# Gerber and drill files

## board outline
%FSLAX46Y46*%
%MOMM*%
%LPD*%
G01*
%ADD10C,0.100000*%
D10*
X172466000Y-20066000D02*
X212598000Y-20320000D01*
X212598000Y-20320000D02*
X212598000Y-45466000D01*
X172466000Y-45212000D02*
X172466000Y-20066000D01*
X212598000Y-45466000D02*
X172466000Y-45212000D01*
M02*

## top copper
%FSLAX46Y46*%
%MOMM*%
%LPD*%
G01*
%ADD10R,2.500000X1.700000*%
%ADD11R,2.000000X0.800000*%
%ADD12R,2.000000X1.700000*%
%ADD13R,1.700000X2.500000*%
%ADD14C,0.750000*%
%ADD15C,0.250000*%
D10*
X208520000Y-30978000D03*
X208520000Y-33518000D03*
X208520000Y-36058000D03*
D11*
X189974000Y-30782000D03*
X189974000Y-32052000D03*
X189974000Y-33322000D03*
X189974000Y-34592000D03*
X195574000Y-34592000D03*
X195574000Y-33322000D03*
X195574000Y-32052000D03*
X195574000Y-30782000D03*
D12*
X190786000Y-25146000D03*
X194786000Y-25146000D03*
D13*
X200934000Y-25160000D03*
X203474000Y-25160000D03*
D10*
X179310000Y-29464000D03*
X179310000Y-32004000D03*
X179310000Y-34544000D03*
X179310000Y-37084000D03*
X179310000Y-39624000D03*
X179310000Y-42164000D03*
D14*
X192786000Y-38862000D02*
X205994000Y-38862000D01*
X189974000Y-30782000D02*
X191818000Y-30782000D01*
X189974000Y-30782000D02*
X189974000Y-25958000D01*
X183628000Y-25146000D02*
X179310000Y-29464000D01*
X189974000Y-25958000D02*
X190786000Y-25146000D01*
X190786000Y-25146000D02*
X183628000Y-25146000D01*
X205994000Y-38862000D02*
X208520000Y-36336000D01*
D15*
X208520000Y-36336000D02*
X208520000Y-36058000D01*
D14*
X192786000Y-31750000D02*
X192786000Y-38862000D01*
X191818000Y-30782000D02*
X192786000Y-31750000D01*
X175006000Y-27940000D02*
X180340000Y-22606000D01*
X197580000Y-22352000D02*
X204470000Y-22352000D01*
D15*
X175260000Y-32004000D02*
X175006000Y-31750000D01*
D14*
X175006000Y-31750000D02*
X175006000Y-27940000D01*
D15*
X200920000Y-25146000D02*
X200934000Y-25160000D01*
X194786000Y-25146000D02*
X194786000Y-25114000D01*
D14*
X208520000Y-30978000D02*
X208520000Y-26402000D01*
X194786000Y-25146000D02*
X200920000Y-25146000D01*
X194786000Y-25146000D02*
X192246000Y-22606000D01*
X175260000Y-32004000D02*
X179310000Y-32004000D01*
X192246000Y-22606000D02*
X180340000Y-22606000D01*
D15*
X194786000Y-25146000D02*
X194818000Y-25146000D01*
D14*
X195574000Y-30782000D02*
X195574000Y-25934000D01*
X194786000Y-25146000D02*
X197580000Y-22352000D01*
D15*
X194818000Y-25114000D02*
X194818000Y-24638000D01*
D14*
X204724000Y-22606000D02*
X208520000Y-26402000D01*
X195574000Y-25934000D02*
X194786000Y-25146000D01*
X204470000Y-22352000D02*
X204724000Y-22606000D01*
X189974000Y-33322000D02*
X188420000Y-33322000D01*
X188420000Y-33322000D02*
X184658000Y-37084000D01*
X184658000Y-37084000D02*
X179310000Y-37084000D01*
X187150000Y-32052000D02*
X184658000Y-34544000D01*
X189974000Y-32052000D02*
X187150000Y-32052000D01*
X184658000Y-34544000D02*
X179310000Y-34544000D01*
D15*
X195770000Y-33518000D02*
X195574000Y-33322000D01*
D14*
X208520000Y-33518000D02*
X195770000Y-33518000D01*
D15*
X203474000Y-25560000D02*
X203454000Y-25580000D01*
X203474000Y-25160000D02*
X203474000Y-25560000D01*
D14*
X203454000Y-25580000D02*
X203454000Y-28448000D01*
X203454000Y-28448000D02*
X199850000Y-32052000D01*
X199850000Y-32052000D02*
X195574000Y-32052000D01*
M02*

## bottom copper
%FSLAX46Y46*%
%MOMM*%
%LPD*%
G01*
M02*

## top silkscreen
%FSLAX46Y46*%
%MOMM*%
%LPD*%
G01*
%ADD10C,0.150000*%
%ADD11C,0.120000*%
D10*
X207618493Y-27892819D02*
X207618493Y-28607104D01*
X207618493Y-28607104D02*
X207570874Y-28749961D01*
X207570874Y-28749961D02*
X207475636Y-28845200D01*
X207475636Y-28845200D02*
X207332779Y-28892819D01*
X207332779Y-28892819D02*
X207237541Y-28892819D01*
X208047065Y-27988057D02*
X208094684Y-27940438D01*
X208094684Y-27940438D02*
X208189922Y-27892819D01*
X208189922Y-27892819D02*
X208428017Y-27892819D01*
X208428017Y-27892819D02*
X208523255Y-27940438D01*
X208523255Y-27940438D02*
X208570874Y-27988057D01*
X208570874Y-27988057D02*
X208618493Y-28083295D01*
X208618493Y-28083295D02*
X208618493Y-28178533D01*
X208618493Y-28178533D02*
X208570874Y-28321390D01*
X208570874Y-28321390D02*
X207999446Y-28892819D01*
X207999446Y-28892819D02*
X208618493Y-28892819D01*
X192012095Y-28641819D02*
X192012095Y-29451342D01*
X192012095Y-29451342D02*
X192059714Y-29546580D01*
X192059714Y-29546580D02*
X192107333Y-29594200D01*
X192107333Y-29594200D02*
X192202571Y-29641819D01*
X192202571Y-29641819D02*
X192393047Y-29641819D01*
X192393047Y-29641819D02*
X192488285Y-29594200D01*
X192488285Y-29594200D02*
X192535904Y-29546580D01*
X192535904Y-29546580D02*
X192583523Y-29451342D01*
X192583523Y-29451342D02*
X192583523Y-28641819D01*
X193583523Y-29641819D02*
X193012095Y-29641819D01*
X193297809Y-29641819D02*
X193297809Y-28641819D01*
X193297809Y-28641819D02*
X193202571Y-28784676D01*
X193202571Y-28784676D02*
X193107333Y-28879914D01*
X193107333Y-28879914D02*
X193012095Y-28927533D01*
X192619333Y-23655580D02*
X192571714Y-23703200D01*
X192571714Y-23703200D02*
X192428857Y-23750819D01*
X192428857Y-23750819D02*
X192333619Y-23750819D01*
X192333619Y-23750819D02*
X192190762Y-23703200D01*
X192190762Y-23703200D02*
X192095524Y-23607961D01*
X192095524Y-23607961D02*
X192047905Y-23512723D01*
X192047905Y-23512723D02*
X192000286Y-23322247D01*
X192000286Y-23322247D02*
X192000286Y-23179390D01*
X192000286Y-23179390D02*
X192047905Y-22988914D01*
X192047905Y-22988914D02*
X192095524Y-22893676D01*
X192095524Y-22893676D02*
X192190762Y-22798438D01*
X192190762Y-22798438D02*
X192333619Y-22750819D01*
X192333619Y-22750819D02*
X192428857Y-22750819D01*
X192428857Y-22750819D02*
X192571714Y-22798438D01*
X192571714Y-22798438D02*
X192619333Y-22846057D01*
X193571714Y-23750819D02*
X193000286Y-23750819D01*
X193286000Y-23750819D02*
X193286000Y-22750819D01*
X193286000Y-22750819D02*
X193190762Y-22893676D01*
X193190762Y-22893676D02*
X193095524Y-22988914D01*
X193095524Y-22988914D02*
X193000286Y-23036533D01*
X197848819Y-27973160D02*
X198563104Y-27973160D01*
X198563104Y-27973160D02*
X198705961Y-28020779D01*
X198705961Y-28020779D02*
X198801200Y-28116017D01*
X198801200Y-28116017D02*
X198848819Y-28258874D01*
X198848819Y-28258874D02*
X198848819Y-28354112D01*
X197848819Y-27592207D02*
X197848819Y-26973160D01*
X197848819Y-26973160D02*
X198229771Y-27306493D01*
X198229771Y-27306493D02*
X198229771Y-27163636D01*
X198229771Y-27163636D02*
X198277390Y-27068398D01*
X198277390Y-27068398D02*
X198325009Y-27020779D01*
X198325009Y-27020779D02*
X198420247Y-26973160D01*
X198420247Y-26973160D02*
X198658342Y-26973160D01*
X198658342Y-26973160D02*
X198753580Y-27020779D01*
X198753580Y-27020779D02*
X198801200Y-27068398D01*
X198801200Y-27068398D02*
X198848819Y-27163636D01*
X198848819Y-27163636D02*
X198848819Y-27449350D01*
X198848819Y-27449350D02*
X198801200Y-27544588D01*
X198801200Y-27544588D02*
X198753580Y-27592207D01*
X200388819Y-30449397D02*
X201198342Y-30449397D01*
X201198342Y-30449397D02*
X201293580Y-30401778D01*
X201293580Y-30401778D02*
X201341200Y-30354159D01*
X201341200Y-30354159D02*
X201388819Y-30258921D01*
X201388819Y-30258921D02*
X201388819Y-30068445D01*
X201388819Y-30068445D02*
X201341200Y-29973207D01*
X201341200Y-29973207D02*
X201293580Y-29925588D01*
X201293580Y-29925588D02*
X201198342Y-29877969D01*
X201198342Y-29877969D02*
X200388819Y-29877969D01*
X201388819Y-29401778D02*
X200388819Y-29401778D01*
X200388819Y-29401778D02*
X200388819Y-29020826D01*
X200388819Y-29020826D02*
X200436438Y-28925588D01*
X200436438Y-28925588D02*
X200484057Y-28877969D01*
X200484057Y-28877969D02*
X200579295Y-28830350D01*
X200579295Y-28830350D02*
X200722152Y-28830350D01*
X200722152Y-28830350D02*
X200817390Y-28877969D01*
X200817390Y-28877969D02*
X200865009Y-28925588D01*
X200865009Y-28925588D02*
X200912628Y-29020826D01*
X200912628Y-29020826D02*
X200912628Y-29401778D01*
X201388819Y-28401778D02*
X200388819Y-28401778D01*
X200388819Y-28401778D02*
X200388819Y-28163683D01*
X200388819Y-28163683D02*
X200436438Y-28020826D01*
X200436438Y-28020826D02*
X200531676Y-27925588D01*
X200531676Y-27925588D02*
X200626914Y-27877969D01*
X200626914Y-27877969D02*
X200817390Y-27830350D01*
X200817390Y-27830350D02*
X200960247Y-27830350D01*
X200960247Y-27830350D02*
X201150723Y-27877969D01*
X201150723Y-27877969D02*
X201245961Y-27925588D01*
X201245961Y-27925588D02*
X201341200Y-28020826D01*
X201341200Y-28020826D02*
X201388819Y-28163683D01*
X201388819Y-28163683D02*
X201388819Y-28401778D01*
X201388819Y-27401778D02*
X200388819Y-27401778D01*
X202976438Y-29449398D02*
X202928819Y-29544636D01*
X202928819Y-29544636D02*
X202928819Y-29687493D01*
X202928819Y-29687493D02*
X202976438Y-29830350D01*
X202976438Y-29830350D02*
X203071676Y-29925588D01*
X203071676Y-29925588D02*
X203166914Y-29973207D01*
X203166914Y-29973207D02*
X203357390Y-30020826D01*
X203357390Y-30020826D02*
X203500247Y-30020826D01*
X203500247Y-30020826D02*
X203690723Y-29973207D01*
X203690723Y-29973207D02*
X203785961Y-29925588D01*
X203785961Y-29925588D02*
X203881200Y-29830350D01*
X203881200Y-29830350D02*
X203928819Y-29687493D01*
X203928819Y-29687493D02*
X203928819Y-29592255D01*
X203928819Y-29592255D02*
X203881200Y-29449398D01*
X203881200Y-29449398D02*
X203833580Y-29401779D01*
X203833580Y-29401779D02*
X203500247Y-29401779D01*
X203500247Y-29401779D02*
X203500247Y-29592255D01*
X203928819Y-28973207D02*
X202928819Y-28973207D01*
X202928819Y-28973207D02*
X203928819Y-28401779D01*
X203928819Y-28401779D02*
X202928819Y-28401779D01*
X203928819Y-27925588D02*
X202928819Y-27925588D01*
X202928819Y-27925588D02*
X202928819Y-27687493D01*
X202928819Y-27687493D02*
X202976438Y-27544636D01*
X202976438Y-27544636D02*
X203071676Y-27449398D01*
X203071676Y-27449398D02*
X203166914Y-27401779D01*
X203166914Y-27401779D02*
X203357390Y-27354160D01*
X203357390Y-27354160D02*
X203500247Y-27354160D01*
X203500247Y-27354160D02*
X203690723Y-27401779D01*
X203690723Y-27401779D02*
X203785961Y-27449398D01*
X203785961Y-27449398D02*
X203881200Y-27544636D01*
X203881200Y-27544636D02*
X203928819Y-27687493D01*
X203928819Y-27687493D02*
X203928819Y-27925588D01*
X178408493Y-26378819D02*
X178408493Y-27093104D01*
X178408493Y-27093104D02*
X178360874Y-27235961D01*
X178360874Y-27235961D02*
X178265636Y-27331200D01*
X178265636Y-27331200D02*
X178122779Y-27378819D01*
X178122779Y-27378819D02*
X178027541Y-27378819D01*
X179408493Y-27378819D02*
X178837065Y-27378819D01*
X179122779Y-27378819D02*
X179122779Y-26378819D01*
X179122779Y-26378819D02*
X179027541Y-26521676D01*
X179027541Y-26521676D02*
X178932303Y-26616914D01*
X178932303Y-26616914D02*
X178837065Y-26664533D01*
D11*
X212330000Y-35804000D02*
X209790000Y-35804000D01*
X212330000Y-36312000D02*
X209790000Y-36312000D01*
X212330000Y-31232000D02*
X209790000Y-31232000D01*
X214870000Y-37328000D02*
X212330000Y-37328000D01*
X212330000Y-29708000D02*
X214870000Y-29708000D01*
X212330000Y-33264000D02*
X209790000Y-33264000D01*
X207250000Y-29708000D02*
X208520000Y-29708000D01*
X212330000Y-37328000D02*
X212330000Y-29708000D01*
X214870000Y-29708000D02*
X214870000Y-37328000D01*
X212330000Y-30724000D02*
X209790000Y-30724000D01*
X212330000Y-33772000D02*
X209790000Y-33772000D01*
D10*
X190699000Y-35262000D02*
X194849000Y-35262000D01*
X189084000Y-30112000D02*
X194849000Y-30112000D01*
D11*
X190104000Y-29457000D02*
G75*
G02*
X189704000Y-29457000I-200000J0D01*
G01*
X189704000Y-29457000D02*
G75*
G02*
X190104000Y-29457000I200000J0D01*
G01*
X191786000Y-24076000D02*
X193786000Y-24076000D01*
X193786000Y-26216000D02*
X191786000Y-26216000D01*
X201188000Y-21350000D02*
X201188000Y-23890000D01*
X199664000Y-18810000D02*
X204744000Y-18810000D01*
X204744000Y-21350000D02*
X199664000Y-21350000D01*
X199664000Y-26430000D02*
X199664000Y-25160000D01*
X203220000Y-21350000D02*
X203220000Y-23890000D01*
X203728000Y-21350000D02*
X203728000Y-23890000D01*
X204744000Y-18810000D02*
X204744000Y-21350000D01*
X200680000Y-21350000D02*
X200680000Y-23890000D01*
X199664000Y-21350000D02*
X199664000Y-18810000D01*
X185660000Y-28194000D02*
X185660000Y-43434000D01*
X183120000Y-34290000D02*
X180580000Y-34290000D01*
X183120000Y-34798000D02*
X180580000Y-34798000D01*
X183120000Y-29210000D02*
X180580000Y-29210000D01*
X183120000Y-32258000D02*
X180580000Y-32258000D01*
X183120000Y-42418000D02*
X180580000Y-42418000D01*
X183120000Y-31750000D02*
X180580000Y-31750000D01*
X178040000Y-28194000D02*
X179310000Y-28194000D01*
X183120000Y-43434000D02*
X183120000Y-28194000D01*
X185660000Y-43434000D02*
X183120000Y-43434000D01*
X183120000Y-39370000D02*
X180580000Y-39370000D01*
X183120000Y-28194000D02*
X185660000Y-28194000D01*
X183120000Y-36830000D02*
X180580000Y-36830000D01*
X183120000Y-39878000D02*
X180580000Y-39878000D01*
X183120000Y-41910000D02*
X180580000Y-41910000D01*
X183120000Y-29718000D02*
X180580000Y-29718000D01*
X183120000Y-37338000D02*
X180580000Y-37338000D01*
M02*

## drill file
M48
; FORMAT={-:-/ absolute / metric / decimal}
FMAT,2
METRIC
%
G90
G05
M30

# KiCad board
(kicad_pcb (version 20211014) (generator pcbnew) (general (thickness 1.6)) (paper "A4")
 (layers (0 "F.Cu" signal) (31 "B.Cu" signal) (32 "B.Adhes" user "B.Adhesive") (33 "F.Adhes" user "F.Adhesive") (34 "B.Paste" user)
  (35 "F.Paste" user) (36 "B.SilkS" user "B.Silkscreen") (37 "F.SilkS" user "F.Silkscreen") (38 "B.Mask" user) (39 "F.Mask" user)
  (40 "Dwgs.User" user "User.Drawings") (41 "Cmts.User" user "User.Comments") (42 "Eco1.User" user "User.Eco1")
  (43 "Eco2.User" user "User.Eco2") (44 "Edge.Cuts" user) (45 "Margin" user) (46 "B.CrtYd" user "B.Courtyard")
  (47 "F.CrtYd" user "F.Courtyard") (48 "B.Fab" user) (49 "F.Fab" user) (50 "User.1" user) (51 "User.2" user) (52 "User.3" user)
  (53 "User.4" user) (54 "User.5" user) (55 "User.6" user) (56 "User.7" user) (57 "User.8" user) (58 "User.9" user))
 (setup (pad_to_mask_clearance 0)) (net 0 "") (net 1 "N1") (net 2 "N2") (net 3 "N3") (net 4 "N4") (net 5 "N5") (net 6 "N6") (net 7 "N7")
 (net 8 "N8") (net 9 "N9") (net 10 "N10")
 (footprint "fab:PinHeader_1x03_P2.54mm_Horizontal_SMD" (layer "F.Cu") (at 208.52 30.978)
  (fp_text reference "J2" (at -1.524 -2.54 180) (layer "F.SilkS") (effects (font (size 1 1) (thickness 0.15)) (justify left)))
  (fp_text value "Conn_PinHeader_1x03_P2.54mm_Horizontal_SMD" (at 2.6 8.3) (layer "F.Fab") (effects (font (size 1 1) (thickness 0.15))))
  (fp_line (start 3.81 4.826) (end 1.27 4.826) (layer "F.SilkS") (width 0.12))
  (fp_line (start 3.81 5.334) (end 1.27 5.334) (layer "F.SilkS") (width 0.12))
  (fp_line (start 3.81 0.254) (end 1.27 0.254) (layer "F.SilkS") (width 0.12))
  (fp_line (start 6.35 6.35) (end 3.81 6.35) (layer "F.SilkS") (width 0.12))
  (fp_line (start 3.81 -1.27) (end 6.35 -1.27) (layer "F.SilkS") (width 0.12))
  (fp_line (start 3.81 2.286) (end 1.27 2.286) (layer "F.SilkS") (width 0.12))
  (fp_line (start -1.27 -1.27) (end 0 -1.27) (layer "F.SilkS") (width 0.12))
  (fp_line (start 3.81 6.35) (end 3.81 -1.27) (layer "F.SilkS") (width 0.12))
  (fp_line (start 6.35 -1.27) (end 6.35 6.35) (layer "F.SilkS") (width 0.12))
  (fp_line (start 3.81 -0.254) (end 1.27 -0.254) (layer "F.SilkS") (width 0.12))
  (fp_line (start 3.81 2.794) (end 1.27 2.794) (layer "F.SilkS") (width 0.12))
  (pad "1" smd rect locked (at 0 0) (size 2.5 1.7) (layers "F.Cu" "F.Paste" "F.Mask") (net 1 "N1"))
  (pad "2" smd rect locked (at 0 2.54) (size 2.5 1.7) (layers "F.Cu" "F.Paste" "F.Mask") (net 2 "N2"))
  (pad "3" smd rect locked (at 0 5.08) (size 2.5 1.7) (layers "F.Cu" "F.Paste" "F.Mask") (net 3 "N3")))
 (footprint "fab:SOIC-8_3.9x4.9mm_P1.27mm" (layer "F.Cu") (at 192.774 32.687)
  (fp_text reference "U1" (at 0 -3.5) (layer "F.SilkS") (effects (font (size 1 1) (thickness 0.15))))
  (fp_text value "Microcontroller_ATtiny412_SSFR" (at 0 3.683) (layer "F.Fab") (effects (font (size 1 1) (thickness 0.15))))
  (fp_line (start -2.075 2.575) (end 2.075 2.575) (layer "F.SilkS") (width 0.15))
  (fp_line (start -3.69 -2.575) (end 2.075 -2.575) (layer "F.SilkS") (width 0.15))
  (fp_circle (center -2.87 -3.23) (end -2.67 -3.23) (layer "F.SilkS") (width 0.12) (fill none))
  (pad "1" smd rect locked (at -2.8 -1.905) (size 2 0.8) (layers "F.Cu" "F.Paste" "F.Mask") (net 3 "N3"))
  (pad "2" smd rect locked (at -2.8 -0.635) (size 2 0.8) (layers "F.Cu" "F.Paste" "F.Mask") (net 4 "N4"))
  (pad "3" smd rect locked (at -2.8 0.635) (size 2 0.8) (layers "F.Cu" "F.Paste" "F.Mask") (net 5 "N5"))
  (pad "4" smd rect locked (at -2.8 1.905) (size 2 0.8) (layers "F.Cu" "F.Paste" "F.Mask") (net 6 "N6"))
  (pad "5" smd rect locked (at 2.8 1.905) (size 2 0.8) (layers "F.Cu" "F.Paste" "F.Mask") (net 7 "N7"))
  (pad "6" smd rect locked (at 2.8 0.635) (size 2 0.8) (layers "F.Cu" "F.Paste" "F.Mask") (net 2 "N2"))
  (pad "7" smd rect locked (at 2.8 -0.635) (size 2 0.8) (layers "F.Cu" "F.Paste" "F.Mask") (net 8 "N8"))
  (pad "8" smd rect locked (at 2.8 -1.905) (size 2 0.8) (layers "F.Cu" "F.Paste" "F.Mask") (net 1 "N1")))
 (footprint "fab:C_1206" (layer "F.Cu") (at 192.786 25.146)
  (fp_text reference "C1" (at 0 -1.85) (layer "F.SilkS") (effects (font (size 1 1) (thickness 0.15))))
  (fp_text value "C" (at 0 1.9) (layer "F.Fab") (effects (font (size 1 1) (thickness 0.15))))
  (fp_line (start -1 -1.07) (end 1 -1.07) (layer "F.SilkS") (width 0.12))
  (fp_line (start 1 1.07) (end -1 1.07) (layer "F.SilkS") (width 0.12))
  (pad "1" smd rect locked (at -2 0) (size 2 1.7) (layers "F.Cu" "F.Paste" "F.Mask") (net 3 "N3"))
  (pad "2" smd rect locked (at 2 0) (size 2 1.7) (layers "F.Cu" "F.Paste" "F.Mask") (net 1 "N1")))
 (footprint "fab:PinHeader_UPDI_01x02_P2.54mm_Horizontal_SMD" (layer "F.Cu") (at 200.934 25.16 90)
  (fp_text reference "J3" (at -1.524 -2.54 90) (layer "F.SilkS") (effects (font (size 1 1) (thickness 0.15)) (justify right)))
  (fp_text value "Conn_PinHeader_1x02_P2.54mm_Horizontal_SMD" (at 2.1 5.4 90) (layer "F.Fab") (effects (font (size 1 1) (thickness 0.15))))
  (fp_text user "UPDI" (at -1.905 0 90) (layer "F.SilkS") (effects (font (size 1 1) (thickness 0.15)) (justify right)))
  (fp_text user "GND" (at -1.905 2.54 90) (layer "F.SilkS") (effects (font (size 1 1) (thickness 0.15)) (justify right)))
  (fp_line (start 3.81 0.254) (end 1.27 0.254) (layer "F.SilkS") (width 0.12))
  (fp_line (start 6.35 -1.27) (end 6.35 3.81) (layer "F.SilkS") (width 0.12))
  (fp_line (start 3.81 3.81) (end 3.81 -1.27) (layer "F.SilkS") (width 0.12))
  (fp_line (start -1.27 -1.27) (end 0 -1.27) (layer "F.SilkS") (width 0.12))
  (fp_line (start 3.81 2.286) (end 1.27 2.286) (layer "F.SilkS") (width 0.12))
  (fp_line (start 3.81 2.794) (end 1.27 2.794) (layer "F.SilkS") (width 0.12))
  (fp_line (start 6.35 3.81) (end 3.81 3.81) (layer "F.SilkS") (width 0.12))
  (fp_line (start 3.81 -0.254) (end 1.27 -0.254) (layer "F.SilkS") (width 0.12))
  (fp_line (start 3.81 -1.27) (end 6.35 -1.27) (layer "F.SilkS") (width 0.12))
  (pad "1" smd rect locked (at 0 0 90) (size 2.5 1.7) (layers "F.Cu" "F.Paste" "F.Mask") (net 1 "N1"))
  (pad "2" smd rect locked (at 0 2.54 90) (size 2.5 1.7) (layers "F.Cu" "F.Paste" "F.Mask") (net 8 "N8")))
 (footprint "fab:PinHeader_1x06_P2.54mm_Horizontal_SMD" (layer "F.Cu") (at 179.31 29.464)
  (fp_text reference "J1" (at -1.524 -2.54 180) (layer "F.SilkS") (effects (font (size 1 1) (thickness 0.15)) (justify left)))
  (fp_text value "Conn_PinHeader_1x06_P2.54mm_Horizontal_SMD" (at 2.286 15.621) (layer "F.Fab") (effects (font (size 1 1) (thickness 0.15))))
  (fp_line (start 6.35 -1.27) (end 6.35 13.97) (layer "F.SilkS") (width 0.12))
  (fp_line (start 3.81 4.826) (end 1.27 4.826) (layer "F.SilkS") (width 0.12))
  (fp_line (start 3.81 5.334) (end 1.27 5.334) (layer "F.SilkS") (width 0.12))
  (fp_line (start 3.81 -0.254) (end 1.27 -0.254) (layer "F.SilkS") (width 0.12))
  (fp_line (start 3.81 2.794) (end 1.27 2.794) (layer "F.SilkS") (width 0.12))
  (fp_line (start 3.81 12.954) (end 1.27 12.954) (layer "F.SilkS") (width 0.12))
  (fp_line (start 3.81 2.286) (end 1.27 2.286) (layer "F.SilkS") (width 0.12))
  (fp_line (start -1.27 -1.27) (end 0 -1.27) (layer "F.SilkS") (width 0.12))
  (fp_line (start 3.81 13.97) (end 3.81 -1.27) (layer "F.SilkS") (width 0.12))
  (fp_line (start 6.35 13.97) (end 3.81 13.97) (layer "F.SilkS") (width 0.12))
  (fp_line (start 3.81 9.906) (end 1.27 9.906) (layer "F.SilkS") (width 0.12))
  (fp_line (start 3.81 -1.27) (end 6.35 -1.27) (layer "F.SilkS") (width 0.12))
  (fp_line (start 3.81 7.366) (end 1.27 7.366) (layer "F.SilkS") (width 0.12))
  (fp_line (start 3.81 10.414) (end 1.27 10.414) (layer "F.SilkS") (width 0.12))
  (fp_line (start 3.81 12.446) (end 1.27 12.446) (layer "F.SilkS") (width 0.12))
  (fp_line (start 3.81 0.254) (end 1.27 0.254) (layer "F.SilkS") (width 0.12))
  (fp_line (start 3.81 7.874) (end 1.27 7.874) (layer "F.SilkS") (width 0.12))
  (pad "1" smd rect locked (at 0 0) (size 2.5 1.7) (layers "F.Cu" "F.Paste" "F.Mask") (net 3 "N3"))
  (pad "2" smd rect locked (at 0 2.54) (size 2.5 1.7) (layers "F.Cu" "F.Paste" "F.Mask") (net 1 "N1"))
  (pad "3" smd rect locked (at 0 5.08) (size 2.5 1.7) (layers "F.Cu" "F.Paste" "F.Mask") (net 4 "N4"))
  (pad "4" smd rect locked (at 0 7.62) (size 2.5 1.7) (layers "F.Cu" "F.Paste" "F.Mask") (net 5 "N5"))
  (pad "5" smd rect locked (at 0 10.16) (size 2.5 1.7) (layers "F.Cu" "F.Paste" "F.Mask") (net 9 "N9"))
  (pad "6" smd rect locked (at 0 12.7) (size 2.5 1.7) (layers "F.Cu" "F.Paste" "F.Mask") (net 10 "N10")))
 (gr_line (start 172.466 20.066) (end 212.598 20.32) (layer "Edge.Cuts") (width 0.1))
 (gr_line (start 212.598 20.32) (end 212.598 45.466) (layer "Edge.Cuts") (width 0.1))
 (gr_line (start 172.466 45.212) (end 172.466 20.066) (layer "Edge.Cuts") (width 0.1))
 (gr_line (start 212.598 45.466) (end 172.466 45.212) (layer "Edge.Cuts") (width 0.1))
 (segment (start 192.786 38.862) (end 205.994 38.862) (width 0.75) (layer "F.Cu") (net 3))
 (segment (start 189.974 30.782) (end 191.818 30.782) (width 0.75) (layer "F.Cu") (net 3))
 (segment (start 189.974 30.782) (end 189.974 25.958) (width 0.75) (layer "F.Cu") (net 3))
 (segment (start 183.628 25.146) (end 179.31 29.464) (width 0.75) (layer "F.Cu") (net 3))
 (segment (start 189.974 25.958) (end 190.786 25.146) (width 0.75) (layer "F.Cu") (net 3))
 (segment (start 190.786 25.146) (end 183.628 25.146) (width 0.75) (layer "F.Cu") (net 3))
 (segment (start 205.994 38.862) (end 208.52 36.336) (width 0.75) (layer "F.Cu") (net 3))
 (segment (start 208.52 36.336) (end 208.52 36.058) (width 0.25) (layer "F.Cu") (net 3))
 (segment (start 192.786 31.75) (end 192.786 38.862) (width 0.75) (layer "F.Cu") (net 3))
 (segment (start 191.818 30.782) (end 192.786 31.75) (width 0.75) (layer "F.Cu") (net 3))
 (segment (start 175.006 27.94) (end 180.34 22.606) (width 0.75) (layer "F.Cu") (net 1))
 (segment (start 197.58 22.352) (end 204.47 22.352) (width 0.75) (layer "F.Cu") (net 1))
 (segment (start 175.26 32.004) (end 175.006 31.75) (width 0.25) (layer "F.Cu") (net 1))
 (segment (start 175.006 31.75) (end 175.006 27.94) (width 0.75) (layer "F.Cu") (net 1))
 (segment (start 200.92 25.146) (end 200.934 25.16) (width 0.25) (layer "F.Cu") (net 1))
 (segment (start 194.786 25.146) (end 194.786 25.114) (width 0.25) (layer "F.Cu") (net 1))
 (segment (start 208.52 30.978) (end 208.52 26.402) (width 0.75) (layer "F.Cu") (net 1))
 (segment (start 194.786 25.146) (end 200.92 25.146) (width 0.75) (layer "F.Cu") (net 1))
 (segment (start 194.786 25.146) (end 192.246 22.606) (width 0.75) (layer "F.Cu") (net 1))
 (segment (start 175.26 32.004) (end 179.31 32.004) (width 0.75) (layer "F.Cu") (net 1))
 (segment (start 192.246 22.606) (end 180.34 22.606) (width 0.75) (layer "F.Cu") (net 1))
 (segment (start 194.786 25.146) (end 194.818 25.146) (width 0.25) (layer "F.Cu") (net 1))
 (segment (start 195.574 30.782) (end 195.574 25.934) (width 0.75) (layer "F.Cu") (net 1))
 (segment (start 194.786 25.146) (end 197.58 22.352) (width 0.75) (layer "F.Cu") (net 1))
 (segment (start 194.818 25.114) (end 194.818 24.638) (width 0.25) (layer "F.Cu") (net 1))
 (segment (start 204.724 22.606) (end 208.52 26.402) (width 0.75) (layer "F.Cu") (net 1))
 (segment (start 195.574 25.934) (end 194.786 25.146) (width 0.75) (layer "F.Cu") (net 1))
 (segment (start 204.47 22.352) (end 204.724 22.606) (width 0.75) (layer "F.Cu") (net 1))
 (segment (start 189.974 33.322) (end 188.42 33.322) (width 0.75) (layer "F.Cu") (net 5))
 (segment (start 188.42 33.322) (end 184.658 37.084) (width 0.75) (layer "F.Cu") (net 5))
 (segment (start 184.658 37.084) (end 179.31 37.084) (width 0.75) (layer "F.Cu") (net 5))
 (segment (start 187.15 32.052) (end 184.658 34.544) (width 0.75) (layer "F.Cu") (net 4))
 (segment (start 189.974 32.052) (end 187.15 32.052) (width 0.75) (layer "F.Cu") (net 4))
 (segment (start 184.658 34.544) (end 179.31 34.544) (width 0.75) (layer "F.Cu") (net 4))
 (segment (start 195.77 33.518) (end 195.574 33.322) (width 0.25) (layer "F.Cu") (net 2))
 (segment (start 208.52 33.518) (end 195.77 33.518) (width 0.75) (layer "F.Cu") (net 2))
 (segment (start 203.474 25.56) (end 203.454 25.58) (width 0.25) (layer "F.Cu") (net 8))
 (segment (start 203.474 25.16) (end 203.474 25.56) (width 0.25) (layer "F.Cu") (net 8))
 (segment (start 203.454 25.58) (end 203.454 28.448) (width 0.75) (layer "F.Cu") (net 8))
 (segment (start 203.454 28.448) (end 199.85 32.052) (width 0.75) (layer "F.Cu") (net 8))
 (segment (start 199.85 32.052) (end 195.574 32.052) (width 0.75) (layer "F.Cu") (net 8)))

